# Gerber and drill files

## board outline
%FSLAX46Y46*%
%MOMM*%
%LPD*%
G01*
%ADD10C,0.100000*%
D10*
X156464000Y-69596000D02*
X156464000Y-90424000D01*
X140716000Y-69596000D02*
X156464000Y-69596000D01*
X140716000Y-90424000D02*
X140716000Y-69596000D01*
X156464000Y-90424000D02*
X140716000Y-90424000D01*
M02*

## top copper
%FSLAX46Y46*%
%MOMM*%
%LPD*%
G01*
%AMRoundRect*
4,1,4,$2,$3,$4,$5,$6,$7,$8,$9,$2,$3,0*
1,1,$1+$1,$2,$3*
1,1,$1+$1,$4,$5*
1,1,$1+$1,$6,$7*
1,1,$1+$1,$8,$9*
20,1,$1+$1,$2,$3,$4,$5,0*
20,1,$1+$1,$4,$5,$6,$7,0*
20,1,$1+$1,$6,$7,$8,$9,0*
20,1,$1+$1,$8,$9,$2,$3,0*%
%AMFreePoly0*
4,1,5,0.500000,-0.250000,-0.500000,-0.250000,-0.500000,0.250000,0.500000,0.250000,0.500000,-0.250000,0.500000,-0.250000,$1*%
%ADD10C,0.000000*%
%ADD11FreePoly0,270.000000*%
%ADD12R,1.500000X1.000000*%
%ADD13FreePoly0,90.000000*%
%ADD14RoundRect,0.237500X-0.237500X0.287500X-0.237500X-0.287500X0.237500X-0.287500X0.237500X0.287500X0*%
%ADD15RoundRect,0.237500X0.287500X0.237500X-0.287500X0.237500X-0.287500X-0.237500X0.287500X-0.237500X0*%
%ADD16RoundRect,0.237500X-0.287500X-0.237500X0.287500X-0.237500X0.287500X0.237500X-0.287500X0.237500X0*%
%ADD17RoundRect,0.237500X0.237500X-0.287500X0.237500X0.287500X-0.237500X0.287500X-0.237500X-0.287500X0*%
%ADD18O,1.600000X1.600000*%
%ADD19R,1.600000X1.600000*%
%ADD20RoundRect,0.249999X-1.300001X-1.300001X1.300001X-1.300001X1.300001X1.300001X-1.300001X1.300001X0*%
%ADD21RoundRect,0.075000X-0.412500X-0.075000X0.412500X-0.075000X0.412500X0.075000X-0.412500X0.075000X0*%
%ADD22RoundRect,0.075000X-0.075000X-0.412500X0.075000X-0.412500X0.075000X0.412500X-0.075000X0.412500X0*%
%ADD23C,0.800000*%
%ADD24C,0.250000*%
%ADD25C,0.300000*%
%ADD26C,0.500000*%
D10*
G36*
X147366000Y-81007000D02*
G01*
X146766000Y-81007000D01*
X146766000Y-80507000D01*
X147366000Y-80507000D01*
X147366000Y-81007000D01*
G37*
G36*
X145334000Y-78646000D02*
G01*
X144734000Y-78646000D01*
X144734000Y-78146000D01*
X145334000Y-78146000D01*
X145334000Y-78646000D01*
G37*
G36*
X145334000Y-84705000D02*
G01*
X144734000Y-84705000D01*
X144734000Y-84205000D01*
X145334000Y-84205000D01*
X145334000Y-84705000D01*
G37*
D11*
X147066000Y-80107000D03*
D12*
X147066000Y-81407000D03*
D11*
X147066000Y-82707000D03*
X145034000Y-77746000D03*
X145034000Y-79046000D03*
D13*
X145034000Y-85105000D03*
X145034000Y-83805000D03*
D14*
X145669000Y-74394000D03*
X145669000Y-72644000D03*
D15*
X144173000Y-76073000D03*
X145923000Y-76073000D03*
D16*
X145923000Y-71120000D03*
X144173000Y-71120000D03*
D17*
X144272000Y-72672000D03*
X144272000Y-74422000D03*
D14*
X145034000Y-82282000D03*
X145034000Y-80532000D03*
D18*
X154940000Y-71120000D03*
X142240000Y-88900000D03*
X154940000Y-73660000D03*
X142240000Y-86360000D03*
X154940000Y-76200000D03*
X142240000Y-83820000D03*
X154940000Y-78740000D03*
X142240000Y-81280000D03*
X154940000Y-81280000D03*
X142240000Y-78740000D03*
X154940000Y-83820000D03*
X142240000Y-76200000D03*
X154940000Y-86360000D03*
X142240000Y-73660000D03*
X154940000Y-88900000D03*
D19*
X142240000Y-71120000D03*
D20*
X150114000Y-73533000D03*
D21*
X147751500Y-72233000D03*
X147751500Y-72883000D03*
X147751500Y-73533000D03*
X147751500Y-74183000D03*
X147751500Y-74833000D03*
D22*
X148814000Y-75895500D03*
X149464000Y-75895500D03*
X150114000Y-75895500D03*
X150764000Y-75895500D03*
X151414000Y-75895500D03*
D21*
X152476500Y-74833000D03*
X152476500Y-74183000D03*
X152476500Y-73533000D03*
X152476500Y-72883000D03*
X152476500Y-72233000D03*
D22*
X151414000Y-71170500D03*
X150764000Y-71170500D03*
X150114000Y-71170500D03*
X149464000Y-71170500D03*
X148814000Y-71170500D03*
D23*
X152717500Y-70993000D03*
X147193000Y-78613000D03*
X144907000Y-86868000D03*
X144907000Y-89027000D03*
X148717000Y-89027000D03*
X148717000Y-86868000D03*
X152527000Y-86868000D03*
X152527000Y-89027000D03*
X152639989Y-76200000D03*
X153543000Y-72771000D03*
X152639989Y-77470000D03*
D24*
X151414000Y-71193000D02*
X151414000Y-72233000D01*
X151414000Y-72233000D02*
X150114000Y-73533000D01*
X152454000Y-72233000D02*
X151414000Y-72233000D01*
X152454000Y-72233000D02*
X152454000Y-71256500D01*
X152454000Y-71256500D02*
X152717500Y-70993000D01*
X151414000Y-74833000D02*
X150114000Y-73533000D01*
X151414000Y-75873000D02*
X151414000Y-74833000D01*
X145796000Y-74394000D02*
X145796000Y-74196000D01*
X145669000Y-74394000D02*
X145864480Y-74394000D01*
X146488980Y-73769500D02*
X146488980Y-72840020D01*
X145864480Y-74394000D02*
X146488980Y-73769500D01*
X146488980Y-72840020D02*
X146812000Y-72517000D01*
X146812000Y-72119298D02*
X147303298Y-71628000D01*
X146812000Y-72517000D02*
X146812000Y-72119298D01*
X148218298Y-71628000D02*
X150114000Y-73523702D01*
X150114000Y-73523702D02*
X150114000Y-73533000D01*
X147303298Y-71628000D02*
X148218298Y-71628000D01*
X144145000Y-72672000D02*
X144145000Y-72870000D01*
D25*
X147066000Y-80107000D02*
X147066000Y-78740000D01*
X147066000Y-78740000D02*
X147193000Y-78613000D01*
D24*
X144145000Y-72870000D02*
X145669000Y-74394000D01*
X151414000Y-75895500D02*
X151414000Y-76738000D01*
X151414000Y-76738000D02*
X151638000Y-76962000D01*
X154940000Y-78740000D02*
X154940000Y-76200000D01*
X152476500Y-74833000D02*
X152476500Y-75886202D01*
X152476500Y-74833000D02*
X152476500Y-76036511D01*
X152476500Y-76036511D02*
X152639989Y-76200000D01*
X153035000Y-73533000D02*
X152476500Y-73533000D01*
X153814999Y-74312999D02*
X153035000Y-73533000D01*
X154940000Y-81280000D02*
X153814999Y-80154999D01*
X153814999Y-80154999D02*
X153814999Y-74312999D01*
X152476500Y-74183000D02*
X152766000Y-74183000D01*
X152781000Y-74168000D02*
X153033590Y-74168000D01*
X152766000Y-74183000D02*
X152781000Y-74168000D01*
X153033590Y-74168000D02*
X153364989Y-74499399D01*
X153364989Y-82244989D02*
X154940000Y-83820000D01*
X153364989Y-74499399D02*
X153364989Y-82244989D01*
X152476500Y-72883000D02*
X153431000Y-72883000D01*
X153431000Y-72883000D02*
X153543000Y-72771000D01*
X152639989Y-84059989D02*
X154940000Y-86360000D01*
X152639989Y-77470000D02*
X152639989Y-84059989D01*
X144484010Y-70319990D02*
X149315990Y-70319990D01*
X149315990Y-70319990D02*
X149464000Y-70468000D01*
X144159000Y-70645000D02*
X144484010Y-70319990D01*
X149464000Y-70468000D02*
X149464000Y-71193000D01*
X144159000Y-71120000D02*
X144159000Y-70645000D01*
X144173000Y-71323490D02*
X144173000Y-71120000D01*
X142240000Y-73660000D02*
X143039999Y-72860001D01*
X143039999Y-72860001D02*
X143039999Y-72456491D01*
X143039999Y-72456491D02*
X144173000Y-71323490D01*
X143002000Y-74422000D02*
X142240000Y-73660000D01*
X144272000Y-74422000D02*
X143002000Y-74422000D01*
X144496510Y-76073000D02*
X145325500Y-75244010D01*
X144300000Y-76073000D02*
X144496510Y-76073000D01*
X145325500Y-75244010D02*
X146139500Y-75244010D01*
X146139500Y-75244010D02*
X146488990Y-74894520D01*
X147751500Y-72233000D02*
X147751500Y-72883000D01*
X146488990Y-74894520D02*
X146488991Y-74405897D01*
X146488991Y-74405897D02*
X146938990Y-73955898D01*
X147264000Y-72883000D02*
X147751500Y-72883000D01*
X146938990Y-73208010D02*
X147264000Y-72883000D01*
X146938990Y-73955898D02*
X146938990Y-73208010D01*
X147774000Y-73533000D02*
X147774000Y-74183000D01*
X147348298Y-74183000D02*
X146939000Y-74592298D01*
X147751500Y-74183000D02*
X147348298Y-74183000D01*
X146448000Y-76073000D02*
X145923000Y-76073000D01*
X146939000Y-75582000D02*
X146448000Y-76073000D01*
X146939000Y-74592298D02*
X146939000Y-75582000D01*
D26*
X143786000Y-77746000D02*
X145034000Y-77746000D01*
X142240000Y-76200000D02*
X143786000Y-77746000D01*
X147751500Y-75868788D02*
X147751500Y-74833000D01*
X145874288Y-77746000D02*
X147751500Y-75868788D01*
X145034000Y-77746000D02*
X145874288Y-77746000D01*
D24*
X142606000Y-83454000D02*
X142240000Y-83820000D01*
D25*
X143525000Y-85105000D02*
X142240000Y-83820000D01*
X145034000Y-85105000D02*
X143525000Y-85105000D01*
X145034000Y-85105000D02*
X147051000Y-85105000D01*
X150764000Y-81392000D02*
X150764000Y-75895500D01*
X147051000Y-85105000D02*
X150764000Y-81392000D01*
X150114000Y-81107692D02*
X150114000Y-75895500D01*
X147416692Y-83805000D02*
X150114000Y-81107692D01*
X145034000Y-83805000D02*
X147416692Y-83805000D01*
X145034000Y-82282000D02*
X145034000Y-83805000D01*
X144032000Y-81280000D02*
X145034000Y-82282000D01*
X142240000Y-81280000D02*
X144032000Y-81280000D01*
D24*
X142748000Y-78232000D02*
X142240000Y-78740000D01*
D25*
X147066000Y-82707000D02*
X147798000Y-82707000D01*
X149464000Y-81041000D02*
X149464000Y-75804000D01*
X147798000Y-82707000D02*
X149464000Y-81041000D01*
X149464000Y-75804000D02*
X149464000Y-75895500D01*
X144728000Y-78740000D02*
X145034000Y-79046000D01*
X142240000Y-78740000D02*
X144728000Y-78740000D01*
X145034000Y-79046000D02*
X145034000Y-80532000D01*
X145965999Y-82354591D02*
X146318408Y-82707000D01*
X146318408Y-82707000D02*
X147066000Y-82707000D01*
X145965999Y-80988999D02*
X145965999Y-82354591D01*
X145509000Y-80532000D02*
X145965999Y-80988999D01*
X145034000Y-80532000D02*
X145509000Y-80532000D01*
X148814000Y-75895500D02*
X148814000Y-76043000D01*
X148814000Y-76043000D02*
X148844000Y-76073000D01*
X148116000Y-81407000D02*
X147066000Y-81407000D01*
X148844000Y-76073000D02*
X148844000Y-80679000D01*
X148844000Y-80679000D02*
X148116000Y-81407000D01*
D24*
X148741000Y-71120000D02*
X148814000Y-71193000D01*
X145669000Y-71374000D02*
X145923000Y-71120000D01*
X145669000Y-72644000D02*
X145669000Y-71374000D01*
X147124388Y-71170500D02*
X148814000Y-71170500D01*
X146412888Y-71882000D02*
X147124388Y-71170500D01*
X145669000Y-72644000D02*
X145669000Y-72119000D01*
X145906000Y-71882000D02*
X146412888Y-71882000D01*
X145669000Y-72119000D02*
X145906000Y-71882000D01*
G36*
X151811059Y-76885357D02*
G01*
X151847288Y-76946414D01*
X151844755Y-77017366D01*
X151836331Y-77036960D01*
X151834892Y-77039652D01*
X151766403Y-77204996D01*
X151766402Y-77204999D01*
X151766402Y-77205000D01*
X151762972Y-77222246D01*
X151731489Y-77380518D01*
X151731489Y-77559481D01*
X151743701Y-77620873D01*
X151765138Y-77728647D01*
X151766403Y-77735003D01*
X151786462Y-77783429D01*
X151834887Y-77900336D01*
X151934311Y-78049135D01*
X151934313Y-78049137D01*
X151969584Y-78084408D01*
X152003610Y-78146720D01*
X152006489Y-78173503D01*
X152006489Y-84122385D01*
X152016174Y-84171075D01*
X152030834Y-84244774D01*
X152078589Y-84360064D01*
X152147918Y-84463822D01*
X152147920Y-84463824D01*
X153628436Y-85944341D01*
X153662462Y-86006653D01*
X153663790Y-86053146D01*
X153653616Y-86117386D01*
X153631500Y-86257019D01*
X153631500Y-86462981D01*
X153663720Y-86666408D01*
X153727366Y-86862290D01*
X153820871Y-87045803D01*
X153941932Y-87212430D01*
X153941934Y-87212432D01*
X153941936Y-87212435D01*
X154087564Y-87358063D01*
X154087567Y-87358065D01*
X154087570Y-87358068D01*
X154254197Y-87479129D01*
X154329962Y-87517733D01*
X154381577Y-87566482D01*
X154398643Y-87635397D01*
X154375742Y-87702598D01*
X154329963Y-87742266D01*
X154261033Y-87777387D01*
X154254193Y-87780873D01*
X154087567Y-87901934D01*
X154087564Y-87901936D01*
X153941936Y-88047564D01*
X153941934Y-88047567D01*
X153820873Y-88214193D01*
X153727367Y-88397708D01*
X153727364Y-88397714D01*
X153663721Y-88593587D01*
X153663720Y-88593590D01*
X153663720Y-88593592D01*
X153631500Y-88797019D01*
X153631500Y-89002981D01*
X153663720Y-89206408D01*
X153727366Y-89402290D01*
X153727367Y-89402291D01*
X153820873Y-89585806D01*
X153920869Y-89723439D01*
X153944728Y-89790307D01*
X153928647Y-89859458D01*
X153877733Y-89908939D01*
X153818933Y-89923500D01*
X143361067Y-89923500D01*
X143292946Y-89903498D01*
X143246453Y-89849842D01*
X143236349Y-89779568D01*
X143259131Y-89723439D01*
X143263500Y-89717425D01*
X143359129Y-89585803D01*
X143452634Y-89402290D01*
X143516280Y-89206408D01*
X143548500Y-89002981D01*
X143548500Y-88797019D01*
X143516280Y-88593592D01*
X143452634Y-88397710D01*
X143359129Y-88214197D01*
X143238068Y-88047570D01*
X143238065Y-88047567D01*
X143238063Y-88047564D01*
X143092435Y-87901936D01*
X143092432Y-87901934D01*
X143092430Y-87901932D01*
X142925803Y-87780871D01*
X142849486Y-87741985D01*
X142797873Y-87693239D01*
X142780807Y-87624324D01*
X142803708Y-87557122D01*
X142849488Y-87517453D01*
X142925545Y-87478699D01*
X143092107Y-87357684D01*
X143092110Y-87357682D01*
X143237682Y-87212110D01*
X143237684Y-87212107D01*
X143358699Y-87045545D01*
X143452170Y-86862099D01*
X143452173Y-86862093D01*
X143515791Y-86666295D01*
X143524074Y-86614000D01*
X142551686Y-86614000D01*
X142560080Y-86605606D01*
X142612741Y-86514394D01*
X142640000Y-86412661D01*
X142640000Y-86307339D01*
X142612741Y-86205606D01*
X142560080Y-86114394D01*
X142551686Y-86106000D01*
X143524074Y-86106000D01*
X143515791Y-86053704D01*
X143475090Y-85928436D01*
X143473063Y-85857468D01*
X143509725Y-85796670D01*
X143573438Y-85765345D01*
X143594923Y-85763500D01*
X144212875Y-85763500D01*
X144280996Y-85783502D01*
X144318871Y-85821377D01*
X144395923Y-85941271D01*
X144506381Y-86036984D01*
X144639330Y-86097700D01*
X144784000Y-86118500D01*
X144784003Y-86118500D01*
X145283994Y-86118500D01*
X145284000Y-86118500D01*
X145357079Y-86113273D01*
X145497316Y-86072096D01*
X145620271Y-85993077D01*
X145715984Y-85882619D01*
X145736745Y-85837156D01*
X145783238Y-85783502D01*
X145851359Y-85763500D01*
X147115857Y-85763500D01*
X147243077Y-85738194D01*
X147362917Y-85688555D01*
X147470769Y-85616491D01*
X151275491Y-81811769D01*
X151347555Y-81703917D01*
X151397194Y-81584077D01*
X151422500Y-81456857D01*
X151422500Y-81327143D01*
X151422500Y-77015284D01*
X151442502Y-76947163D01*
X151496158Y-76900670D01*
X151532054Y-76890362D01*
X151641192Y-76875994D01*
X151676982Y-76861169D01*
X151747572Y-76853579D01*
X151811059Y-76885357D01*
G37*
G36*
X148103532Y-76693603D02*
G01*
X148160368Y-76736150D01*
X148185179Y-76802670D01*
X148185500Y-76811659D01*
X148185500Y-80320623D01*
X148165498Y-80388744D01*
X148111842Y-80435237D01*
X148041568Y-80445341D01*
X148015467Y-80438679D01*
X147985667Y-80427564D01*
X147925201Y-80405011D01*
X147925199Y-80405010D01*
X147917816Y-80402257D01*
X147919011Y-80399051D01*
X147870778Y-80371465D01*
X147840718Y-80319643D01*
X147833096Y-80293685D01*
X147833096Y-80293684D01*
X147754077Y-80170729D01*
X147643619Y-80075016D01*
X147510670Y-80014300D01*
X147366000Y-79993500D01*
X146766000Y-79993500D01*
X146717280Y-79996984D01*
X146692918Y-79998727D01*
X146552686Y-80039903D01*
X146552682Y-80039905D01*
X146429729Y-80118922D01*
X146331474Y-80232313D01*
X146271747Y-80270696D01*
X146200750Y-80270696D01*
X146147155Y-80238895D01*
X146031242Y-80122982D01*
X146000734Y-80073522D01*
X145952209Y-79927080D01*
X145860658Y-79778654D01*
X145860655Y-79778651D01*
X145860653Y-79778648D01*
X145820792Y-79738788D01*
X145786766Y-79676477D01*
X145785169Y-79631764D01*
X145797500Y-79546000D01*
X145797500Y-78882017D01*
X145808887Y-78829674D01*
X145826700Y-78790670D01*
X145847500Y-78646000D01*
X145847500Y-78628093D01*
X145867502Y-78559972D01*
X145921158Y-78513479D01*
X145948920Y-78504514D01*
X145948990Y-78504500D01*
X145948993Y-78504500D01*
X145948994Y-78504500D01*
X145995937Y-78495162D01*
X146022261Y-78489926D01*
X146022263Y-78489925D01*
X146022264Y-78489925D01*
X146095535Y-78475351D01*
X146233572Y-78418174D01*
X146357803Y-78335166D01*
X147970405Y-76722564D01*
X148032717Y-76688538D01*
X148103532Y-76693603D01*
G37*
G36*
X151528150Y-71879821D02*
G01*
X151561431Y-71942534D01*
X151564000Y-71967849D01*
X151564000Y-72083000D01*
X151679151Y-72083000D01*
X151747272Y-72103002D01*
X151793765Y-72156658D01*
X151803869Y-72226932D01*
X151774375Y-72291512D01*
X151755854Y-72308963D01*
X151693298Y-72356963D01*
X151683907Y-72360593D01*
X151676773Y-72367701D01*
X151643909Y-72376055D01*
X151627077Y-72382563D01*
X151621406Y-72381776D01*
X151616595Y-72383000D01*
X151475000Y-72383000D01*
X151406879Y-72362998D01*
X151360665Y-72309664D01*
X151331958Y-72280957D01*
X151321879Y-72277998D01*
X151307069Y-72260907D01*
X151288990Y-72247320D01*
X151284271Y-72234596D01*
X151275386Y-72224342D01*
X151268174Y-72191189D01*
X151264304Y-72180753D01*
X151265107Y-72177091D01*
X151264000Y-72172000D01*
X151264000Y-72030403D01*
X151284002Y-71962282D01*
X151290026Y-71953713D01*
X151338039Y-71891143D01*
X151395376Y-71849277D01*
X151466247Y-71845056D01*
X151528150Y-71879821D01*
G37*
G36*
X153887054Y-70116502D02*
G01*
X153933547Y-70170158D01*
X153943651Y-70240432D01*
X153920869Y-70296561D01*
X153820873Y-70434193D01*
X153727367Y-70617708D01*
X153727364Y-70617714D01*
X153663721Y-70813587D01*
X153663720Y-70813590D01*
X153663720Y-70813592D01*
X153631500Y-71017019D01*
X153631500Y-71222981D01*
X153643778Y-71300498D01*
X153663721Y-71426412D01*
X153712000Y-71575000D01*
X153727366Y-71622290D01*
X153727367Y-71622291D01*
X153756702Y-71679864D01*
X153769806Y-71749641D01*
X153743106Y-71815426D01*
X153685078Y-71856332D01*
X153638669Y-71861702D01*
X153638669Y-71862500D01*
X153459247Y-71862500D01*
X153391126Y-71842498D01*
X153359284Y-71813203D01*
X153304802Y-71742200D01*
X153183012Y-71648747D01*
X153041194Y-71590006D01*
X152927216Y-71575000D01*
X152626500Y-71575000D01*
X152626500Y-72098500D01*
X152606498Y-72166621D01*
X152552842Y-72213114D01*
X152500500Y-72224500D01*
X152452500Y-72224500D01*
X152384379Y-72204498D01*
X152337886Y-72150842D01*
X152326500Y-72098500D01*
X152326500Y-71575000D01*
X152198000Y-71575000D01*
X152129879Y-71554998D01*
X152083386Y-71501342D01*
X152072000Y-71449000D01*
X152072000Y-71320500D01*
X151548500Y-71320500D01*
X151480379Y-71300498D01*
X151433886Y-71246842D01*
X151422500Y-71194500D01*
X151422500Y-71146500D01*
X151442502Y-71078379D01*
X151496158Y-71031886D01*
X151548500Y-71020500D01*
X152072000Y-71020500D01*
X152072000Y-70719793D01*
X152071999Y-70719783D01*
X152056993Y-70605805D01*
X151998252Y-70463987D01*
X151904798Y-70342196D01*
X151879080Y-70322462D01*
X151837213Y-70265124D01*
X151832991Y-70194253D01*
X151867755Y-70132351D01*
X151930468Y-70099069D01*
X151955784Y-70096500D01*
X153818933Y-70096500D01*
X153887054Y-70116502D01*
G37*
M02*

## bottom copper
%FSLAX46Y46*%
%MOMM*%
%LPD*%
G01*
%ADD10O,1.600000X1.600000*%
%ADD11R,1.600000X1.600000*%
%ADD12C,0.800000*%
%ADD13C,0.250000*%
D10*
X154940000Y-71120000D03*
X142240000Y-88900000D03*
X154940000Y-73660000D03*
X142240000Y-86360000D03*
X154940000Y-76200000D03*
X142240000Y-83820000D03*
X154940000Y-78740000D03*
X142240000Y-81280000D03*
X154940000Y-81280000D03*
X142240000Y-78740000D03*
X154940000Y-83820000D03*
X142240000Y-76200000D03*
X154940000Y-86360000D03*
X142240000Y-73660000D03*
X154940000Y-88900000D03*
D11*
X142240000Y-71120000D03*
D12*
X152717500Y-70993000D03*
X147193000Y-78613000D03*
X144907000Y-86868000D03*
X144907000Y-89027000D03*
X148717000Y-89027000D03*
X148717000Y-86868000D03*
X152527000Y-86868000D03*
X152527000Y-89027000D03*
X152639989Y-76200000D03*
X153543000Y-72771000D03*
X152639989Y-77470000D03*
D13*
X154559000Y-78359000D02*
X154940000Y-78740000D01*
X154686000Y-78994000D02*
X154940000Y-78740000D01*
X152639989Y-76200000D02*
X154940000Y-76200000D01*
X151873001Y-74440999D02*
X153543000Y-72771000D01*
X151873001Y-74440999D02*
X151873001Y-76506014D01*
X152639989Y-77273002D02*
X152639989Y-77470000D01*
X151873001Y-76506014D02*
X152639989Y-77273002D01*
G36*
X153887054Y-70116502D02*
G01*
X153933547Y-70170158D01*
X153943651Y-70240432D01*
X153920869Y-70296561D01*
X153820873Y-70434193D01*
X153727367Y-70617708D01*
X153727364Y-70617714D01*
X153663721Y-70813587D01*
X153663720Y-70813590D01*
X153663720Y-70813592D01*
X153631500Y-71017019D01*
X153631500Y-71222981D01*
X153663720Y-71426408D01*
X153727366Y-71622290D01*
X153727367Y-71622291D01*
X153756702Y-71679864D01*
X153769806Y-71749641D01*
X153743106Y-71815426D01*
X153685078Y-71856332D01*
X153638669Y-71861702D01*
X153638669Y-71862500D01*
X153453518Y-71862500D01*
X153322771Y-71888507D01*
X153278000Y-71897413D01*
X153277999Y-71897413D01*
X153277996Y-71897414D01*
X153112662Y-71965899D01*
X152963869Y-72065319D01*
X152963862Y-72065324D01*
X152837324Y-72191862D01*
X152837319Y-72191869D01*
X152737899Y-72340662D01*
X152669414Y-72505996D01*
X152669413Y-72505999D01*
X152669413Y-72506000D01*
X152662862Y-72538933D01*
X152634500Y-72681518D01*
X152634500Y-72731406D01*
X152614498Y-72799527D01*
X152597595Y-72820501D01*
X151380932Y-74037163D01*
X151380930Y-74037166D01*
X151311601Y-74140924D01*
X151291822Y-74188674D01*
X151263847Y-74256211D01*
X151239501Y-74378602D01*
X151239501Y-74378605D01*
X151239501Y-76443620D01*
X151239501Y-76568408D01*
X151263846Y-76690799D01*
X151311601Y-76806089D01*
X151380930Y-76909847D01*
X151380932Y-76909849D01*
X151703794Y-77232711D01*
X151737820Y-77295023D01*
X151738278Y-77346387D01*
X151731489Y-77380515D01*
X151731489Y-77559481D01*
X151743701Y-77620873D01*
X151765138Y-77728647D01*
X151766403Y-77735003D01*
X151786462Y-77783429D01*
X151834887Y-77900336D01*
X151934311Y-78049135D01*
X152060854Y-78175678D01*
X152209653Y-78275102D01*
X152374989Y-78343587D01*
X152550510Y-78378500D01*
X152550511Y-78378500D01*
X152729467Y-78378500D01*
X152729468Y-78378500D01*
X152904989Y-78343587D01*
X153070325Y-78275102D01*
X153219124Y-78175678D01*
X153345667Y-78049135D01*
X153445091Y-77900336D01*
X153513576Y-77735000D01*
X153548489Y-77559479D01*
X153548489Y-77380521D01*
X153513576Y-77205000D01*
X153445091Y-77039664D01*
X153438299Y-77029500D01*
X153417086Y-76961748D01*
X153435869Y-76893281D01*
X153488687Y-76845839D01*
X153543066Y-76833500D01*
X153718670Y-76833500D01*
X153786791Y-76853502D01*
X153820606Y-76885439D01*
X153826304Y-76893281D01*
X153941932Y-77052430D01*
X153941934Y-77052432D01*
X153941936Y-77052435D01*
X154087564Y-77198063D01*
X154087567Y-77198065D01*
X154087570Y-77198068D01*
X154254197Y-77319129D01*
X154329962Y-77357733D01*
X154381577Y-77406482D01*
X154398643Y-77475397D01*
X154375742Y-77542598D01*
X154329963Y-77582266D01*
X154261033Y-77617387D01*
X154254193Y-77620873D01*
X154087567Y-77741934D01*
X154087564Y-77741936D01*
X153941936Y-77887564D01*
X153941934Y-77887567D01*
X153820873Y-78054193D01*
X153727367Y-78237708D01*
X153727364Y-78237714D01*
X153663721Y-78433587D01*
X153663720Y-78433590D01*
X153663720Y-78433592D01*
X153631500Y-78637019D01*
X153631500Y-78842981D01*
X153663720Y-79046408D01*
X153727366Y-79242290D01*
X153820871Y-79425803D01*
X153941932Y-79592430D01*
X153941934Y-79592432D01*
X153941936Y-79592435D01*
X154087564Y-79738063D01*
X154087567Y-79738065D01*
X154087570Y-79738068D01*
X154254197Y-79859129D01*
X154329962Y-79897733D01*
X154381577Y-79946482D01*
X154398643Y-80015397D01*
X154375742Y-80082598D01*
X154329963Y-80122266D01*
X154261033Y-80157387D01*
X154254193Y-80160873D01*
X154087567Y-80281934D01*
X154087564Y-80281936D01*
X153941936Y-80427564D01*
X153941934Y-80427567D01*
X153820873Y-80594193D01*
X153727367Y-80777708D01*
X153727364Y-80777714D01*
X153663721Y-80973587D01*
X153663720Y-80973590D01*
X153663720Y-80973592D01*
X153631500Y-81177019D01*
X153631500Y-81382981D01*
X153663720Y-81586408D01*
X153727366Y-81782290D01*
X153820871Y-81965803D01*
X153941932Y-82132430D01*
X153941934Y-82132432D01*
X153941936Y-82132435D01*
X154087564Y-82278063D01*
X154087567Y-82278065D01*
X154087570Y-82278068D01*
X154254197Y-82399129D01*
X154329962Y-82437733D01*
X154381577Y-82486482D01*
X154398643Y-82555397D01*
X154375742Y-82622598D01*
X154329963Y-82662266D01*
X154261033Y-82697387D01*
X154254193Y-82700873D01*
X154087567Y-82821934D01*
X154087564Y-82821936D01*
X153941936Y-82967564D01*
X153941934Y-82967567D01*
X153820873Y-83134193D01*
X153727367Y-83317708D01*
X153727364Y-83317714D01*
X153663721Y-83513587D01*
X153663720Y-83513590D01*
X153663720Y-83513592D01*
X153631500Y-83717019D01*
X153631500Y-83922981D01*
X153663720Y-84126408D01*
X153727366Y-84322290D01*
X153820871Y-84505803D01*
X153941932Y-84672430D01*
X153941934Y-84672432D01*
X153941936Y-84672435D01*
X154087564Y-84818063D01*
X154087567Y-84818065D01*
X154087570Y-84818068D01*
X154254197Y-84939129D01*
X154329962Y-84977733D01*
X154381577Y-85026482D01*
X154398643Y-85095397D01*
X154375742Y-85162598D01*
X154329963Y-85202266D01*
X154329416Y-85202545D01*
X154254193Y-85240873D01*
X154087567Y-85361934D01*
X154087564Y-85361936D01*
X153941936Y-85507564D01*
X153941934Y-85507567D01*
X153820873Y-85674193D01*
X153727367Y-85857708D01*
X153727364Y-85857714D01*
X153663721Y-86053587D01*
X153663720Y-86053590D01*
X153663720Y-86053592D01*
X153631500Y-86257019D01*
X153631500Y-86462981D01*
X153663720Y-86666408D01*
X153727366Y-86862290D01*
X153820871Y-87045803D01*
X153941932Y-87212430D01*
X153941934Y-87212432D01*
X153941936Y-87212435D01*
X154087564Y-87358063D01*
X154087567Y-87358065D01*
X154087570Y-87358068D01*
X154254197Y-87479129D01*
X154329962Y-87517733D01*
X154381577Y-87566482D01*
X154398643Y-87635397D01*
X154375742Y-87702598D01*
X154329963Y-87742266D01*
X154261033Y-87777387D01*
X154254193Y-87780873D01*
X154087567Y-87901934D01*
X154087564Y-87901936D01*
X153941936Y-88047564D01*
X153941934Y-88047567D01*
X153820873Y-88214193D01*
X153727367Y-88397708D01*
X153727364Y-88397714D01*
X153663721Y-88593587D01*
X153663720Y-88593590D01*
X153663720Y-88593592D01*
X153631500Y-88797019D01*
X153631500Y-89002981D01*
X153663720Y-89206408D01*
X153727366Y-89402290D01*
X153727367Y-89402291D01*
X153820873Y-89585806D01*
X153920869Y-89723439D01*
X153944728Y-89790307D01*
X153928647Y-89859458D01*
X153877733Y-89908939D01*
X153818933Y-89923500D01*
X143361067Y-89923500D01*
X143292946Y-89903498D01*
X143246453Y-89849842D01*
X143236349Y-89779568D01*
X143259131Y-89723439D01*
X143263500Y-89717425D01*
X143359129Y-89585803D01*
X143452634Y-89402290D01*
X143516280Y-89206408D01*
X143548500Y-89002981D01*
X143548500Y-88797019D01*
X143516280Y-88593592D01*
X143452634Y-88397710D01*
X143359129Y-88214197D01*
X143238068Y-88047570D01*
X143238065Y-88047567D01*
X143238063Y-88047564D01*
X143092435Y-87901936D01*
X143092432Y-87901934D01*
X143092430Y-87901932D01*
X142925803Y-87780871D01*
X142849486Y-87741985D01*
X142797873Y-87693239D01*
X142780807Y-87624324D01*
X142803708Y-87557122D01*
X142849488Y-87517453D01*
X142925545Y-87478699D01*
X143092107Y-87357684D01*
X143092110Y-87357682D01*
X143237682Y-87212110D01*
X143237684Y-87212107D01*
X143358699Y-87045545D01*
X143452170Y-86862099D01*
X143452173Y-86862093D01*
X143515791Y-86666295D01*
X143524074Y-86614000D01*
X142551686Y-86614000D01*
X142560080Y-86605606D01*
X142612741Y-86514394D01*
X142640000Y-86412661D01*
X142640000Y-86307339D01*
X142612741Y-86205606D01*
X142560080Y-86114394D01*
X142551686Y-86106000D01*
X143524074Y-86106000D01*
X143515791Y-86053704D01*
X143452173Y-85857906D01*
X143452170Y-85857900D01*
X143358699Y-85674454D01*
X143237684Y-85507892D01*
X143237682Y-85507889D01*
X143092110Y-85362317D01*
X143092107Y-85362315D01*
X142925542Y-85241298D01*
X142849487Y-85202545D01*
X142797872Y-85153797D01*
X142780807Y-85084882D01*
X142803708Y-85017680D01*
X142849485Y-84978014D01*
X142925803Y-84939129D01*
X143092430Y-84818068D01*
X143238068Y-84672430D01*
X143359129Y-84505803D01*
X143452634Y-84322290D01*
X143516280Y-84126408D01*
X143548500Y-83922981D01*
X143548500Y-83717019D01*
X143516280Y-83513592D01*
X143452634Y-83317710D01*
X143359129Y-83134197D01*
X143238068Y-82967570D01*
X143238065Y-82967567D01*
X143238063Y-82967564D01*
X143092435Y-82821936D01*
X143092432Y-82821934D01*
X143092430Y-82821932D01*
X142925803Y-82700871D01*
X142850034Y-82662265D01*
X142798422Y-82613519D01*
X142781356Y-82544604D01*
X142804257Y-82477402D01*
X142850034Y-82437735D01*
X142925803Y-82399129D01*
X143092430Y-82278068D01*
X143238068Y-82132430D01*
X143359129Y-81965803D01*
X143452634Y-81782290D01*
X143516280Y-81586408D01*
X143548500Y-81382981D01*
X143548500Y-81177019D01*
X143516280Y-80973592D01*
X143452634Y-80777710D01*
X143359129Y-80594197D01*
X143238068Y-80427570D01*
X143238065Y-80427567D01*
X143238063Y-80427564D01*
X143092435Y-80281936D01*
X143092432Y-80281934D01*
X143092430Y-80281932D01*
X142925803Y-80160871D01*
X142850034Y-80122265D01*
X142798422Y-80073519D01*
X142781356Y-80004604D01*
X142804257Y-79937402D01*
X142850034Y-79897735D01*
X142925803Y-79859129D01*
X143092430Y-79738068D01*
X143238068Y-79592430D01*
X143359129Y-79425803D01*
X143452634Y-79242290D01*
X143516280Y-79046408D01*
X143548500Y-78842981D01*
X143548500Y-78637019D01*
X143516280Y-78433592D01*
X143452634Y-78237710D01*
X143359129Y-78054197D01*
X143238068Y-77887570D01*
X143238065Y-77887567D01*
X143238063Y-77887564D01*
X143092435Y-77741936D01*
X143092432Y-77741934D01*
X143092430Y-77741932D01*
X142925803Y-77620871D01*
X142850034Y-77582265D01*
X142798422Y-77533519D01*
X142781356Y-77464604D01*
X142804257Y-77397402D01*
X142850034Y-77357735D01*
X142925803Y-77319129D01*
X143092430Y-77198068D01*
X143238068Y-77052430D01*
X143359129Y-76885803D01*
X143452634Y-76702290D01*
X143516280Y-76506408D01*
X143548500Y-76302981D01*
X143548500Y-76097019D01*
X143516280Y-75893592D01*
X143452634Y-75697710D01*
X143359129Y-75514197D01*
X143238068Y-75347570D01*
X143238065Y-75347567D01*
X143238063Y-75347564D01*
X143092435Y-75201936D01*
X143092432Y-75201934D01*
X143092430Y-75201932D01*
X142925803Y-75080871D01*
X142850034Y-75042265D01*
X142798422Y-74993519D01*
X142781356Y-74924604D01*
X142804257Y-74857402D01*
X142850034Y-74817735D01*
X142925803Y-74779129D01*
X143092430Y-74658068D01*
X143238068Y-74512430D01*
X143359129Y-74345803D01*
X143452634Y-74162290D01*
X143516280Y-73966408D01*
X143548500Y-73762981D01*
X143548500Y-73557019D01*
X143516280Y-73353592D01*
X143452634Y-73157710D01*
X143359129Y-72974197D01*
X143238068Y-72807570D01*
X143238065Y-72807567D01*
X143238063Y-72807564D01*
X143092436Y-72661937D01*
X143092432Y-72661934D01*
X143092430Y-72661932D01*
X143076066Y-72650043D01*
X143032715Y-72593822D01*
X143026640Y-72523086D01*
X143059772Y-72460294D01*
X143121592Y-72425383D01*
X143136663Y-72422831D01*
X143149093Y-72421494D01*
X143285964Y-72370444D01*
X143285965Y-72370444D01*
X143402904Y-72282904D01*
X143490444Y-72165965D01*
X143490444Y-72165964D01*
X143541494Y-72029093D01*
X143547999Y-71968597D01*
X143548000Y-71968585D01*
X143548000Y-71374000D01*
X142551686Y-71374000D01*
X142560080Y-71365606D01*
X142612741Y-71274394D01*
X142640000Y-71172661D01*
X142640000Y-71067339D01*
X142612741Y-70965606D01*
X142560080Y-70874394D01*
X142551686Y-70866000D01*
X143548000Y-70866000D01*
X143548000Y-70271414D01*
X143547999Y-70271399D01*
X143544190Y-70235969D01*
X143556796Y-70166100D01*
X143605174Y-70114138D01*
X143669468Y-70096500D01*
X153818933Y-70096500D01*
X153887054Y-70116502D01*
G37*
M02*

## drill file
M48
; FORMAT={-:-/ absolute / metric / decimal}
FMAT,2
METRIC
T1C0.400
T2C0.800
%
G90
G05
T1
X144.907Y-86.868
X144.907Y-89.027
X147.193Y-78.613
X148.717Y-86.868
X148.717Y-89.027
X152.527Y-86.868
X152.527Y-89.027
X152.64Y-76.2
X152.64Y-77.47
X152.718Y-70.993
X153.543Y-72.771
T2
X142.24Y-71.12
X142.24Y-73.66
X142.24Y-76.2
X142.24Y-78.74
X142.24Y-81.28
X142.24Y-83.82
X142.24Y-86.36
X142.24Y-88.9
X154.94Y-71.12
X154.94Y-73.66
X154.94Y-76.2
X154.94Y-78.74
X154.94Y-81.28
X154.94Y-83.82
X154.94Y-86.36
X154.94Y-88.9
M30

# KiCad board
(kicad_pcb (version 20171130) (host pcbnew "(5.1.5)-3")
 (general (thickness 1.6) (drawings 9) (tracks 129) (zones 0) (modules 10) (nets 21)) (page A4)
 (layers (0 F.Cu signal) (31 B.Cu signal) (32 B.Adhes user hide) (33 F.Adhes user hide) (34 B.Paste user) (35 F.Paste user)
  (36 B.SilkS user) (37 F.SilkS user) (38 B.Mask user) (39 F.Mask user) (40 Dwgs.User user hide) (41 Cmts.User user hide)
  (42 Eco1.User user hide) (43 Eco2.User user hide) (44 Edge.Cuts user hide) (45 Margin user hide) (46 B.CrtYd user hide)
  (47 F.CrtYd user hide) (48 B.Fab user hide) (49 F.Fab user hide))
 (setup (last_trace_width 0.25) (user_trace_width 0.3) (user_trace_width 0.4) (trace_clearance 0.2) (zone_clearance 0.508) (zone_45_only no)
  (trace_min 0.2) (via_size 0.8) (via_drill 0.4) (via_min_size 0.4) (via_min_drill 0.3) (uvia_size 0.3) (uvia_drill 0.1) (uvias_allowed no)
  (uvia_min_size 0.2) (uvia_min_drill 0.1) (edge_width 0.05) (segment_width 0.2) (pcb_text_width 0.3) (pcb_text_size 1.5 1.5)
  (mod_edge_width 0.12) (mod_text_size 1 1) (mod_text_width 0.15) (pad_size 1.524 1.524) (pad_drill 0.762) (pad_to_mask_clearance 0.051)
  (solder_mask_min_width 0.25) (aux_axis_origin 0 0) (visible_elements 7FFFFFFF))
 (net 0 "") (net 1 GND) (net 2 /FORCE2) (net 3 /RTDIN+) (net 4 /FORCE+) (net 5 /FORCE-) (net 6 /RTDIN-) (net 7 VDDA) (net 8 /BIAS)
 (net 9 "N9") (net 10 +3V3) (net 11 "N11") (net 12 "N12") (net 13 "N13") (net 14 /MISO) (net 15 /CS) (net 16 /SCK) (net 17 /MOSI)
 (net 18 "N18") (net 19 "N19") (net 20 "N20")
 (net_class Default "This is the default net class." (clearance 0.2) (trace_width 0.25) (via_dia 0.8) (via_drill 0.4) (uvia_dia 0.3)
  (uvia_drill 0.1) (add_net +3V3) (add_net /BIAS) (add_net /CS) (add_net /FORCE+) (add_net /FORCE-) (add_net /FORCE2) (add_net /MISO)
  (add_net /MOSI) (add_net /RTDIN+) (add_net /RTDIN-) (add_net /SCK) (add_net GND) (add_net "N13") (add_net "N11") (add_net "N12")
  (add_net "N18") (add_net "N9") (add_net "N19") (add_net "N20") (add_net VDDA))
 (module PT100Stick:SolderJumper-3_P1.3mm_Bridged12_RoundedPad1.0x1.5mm (layer F.Cu) (at 147.066 81.407 270)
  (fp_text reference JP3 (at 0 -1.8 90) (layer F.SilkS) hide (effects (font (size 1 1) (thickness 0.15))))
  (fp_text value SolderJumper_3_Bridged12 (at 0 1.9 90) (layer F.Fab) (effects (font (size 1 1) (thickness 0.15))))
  (fp_poly (pts (xy -0.9 -0.3) (xy -0.4 -0.3) (xy -0.4 0.3) (xy -0.9 0.3)) (layer F.Cu) (width 0))
  (pad 1 smd custom (at -1.3 0 270) (size 1 0.5) (layers F.Cu F.Mask) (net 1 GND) (zone_connect 2)
   (options (clearance outline) (anchor rect)) (primitives))
  (pad 2 smd rect (at 0 0 270) (size 1 1.5) (layers F.Cu F.Mask) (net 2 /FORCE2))
  (pad 3 smd custom (at 1.3 0 270) (size 1 0.5) (layers F.Cu F.Mask) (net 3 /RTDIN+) (zone_connect 2)
   (options (clearance outline) (anchor rect)) (primitives)))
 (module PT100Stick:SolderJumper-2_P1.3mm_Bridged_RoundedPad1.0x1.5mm (layer F.Cu) (at 145.034 78.396 270)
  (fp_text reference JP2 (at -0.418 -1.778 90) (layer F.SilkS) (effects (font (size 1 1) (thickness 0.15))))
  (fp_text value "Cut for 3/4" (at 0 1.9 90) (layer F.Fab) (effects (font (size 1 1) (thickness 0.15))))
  (fp_poly (pts (xy 0.25 -0.3) (xy -0.25 -0.3) (xy -0.25 0.3) (xy 0.25 0.3)) (layer F.Cu) (width 0))
  (pad 1 smd custom (at -0.65 0 270) (size 1 0.5) (layers F.Cu F.Mask) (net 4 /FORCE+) (zone_connect 2)
   (options (clearance outline) (anchor rect)) (primitives))
  (pad 2 smd custom (at 0.65 0 270) (size 1 0.5) (layers F.Cu F.Mask) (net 3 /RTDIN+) (zone_connect 2)
   (options (clearance outline) (anchor rect)) (primitives)))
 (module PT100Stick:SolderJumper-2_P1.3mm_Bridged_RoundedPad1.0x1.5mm (layer F.Cu) (at 145.034 84.455 90)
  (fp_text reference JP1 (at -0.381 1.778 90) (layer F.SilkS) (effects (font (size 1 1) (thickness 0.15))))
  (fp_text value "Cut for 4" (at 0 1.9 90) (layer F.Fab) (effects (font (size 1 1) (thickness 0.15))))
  (fp_poly (pts (xy 0.25 -0.3) (xy -0.25 -0.3) (xy -0.25 0.3) (xy 0.25 0.3)) (layer F.Cu) (width 0))
  (pad 1 smd custom (at -0.65 0 90) (size 1 0.5) (layers F.Cu F.Mask) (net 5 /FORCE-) (zone_connect 2)
   (options (clearance outline) (anchor rect)) (primitives))
  (pad 2 smd custom (at 0.65 0 90) (size 1 0.5) (layers F.Cu F.Mask) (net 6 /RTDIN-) (zone_connect 2)
   (options (clearance outline) (anchor rect)) (primitives)))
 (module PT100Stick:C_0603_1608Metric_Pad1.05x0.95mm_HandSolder (layer F.Cu) (at 145.669 73.519 270)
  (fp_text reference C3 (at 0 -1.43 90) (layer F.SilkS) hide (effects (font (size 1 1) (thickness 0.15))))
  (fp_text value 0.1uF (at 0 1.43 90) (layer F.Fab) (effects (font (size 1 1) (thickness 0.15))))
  (pad 2 smd roundrect (at 0.875 0 270) (size 1.05 0.95) (layers F.Cu F.Paste F.Mask) (roundrect_rratio 0.25) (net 1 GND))
  (pad 1 smd roundrect (at -0.875 0 270) (size 1.05 0.95) (layers F.Cu F.Paste F.Mask) (roundrect_rratio 0.25) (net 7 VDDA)))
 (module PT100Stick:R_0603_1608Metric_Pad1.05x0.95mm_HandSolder (layer F.Cu) (at 145.048 76.073 180)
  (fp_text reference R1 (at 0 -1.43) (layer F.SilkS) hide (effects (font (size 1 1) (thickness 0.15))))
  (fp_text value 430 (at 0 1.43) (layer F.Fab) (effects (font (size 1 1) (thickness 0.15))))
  (pad 2 smd roundrect (at 0.875 0 180) (size 1.05 0.95) (layers F.Cu F.Paste F.Mask) (roundrect_rratio 0.25) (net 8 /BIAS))
  (pad 1 smd roundrect (at -0.875 0 180) (size 1.05 0.95) (layers F.Cu F.Paste F.Mask) (roundrect_rratio 0.25) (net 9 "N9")))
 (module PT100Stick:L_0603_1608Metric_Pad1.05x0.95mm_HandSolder (layer F.Cu) (at 145.048 71.12)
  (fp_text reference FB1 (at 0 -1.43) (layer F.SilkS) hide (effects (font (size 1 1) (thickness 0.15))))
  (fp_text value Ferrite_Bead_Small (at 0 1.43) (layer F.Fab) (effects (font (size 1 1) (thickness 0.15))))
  (pad 2 smd roundrect (at 0.875 0) (size 1.05 0.95) (layers F.Cu F.Paste F.Mask) (roundrect_rratio 0.25) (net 7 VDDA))
  (pad 1 smd roundrect (at -0.875 0) (size 1.05 0.95) (layers F.Cu F.Paste F.Mask) (roundrect_rratio 0.25) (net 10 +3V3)))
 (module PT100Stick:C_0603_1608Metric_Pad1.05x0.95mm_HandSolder (layer F.Cu) (at 144.272 73.547 90)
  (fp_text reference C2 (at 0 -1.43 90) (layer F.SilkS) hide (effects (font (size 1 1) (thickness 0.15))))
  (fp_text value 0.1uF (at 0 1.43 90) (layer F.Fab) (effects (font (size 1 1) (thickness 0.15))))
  (pad 2 smd roundrect (at 0.875 0 90) (size 1.05 0.95) (layers F.Cu F.Paste F.Mask) (roundrect_rratio 0.25) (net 1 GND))
  (pad 1 smd roundrect (at -0.875 0 90) (size 1.05 0.95) (layers F.Cu F.Paste F.Mask) (roundrect_rratio 0.25) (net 10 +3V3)))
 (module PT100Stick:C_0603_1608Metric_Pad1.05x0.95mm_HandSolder (layer F.Cu) (at 145.034 81.407 270)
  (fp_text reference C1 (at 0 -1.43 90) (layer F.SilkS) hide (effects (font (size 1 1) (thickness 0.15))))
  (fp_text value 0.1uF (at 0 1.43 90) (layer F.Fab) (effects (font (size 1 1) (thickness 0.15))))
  (pad 2 smd roundrect (at 0.875 0 270) (size 1.05 0.95) (layers F.Cu F.Paste F.Mask) (roundrect_rratio 0.25) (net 6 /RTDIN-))
  (pad 1 smd roundrect (at -0.875 0 270) (size 1.05 0.95) (layers F.Cu F.Paste F.Mask) (roundrect_rratio 0.25) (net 3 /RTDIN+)))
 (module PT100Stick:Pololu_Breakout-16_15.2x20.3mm (layer F.Cu) (at 142.24 71.12)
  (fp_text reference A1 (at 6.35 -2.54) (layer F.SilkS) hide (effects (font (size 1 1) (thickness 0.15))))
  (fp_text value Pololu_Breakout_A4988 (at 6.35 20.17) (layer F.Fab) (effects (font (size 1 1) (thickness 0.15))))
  (pad 16 thru_hole oval (at 12.7 0) (size 1.6 1.6) (drill 0.8) (layers *.Cu *.Mask) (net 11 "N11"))
  (pad 8 thru_hole oval (at 0 17.78) (size 1.6 1.6) (drill 0.8) (layers *.Cu *.Mask) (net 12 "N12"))
  (pad 15 thru_hole oval (at 12.7 2.54) (size 1.6 1.6) (drill 0.8) (layers *.Cu *.Mask) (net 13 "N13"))
  (pad 7 thru_hole oval (at 0 15.24) (size 1.6 1.6) (drill 0.8) (layers *.Cu *.Mask) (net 1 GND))
  (pad 14 thru_hole oval (at 12.7 5.08) (size 1.6 1.6) (drill 0.8) (layers *.Cu *.Mask) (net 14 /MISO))
  (pad 6 thru_hole oval (at 0 12.7) (size 1.6 1.6) (drill 0.8) (layers *.Cu *.Mask) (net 5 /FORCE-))
  (pad 13 thru_hole oval (at 12.7 7.62) (size 1.6 1.6) (drill 0.8) (layers *.Cu *.Mask) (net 14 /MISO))
  (pad 5 thru_hole oval (at 0 10.16) (size 1.6 1.6) (drill 0.8) (layers *.Cu *.Mask) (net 6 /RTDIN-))
  (pad 12 thru_hole oval (at 12.7 10.16) (size 1.6 1.6) (drill 0.8) (layers *.Cu *.Mask) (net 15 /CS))
  (pad 4 thru_hole oval (at 0 7.62) (size 1.6 1.6) (drill 0.8) (layers *.Cu *.Mask) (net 3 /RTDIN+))
  (pad 11 thru_hole oval (at 12.7 12.7) (size 1.6 1.6) (drill 0.8) (layers *.Cu *.Mask) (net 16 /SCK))
  (pad 3 thru_hole oval (at 0 5.08) (size 1.6 1.6) (drill 0.8) (layers *.Cu *.Mask) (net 4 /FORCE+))
  (pad 10 thru_hole oval (at 12.7 15.24) (size 1.6 1.6) (drill 0.8) (layers *.Cu *.Mask) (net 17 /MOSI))
  (pad 2 thru_hole oval (at 0 2.54) (size 1.6 1.6) (drill 0.8) (layers *.Cu *.Mask) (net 10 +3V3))
  (pad 9 thru_hole oval (at 12.7 17.78) (size 1.6 1.6) (drill 0.8) (layers *.Cu *.Mask) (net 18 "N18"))
  (pad 1 thru_hole rect (at 0 0) (size 1.6 1.6) (drill 0.8) (layers *.Cu *.Mask) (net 1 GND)))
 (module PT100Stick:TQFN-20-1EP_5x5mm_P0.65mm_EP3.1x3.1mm (layer F.Cu) (at 150.114 73.533)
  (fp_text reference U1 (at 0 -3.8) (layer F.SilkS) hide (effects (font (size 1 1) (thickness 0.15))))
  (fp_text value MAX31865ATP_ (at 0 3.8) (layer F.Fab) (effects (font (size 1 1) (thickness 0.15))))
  (pad 21 smd roundrect (at 0 0) (size 3.1 3.1) (layers F.Cu F.Mask) (roundrect_rratio 0.08064499999999999) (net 1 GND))
  (pad "" smd roundrect (at -0.775 -0.775) (size 1.25 1.25) (layers F.Paste) (roundrect_rratio 0.2))
  (pad "" smd roundrect (at -0.775 0.775) (size 1.25 1.25) (layers F.Paste) (roundrect_rratio 0.2))
  (pad "" smd roundrect (at 0.775 -0.775) (size 1.25 1.25) (layers F.Paste) (roundrect_rratio 0.2))
  (pad "" smd roundrect (at 0.775 0.775) (size 1.25 1.25) (layers F.Paste) (roundrect_rratio 0.2))
  (pad 1 smd roundrect (at -2.3625 -1.3) (size 0.975 0.3) (layers F.Cu F.Paste F.Mask) (roundrect_rratio 0.25) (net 8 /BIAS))
  (pad 2 smd roundrect (at -2.3625 -0.65) (size 0.975 0.3) (layers F.Cu F.Paste F.Mask) (roundrect_rratio 0.25) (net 8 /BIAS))
  (pad 3 smd roundrect (at -2.3625 0) (size 0.975 0.3) (layers F.Cu F.Paste F.Mask) (roundrect_rratio 0.25) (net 9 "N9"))
  (pad 4 smd roundrect (at -2.3625 0.65) (size 0.975 0.3) (layers F.Cu F.Paste F.Mask) (roundrect_rratio 0.25) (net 9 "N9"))
  (pad 5 smd roundrect (at -2.3625 1.3) (size 0.975 0.3) (layers F.Cu F.Paste F.Mask) (roundrect_rratio 0.25) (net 4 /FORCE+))
  (pad 6 smd roundrect (at -1.3 2.3625) (size 0.3 0.975) (layers F.Cu F.Paste F.Mask) (roundrect_rratio 0.25) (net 2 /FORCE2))
  (pad 7 smd roundrect (at -0.65 2.3625) (size 0.3 0.975) (layers F.Cu F.Paste F.Mask) (roundrect_rratio 0.25) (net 3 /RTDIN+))
  (pad 8 smd roundrect (at 0 2.3625) (size 0.3 0.975) (layers F.Cu F.Paste F.Mask) (roundrect_rratio 0.25) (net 6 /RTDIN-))
  (pad 9 smd roundrect (at 0.65 2.3625) (size 0.3 0.975) (layers F.Cu F.Paste F.Mask) (roundrect_rratio 0.25) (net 5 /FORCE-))
  (pad 10 smd roundrect (at 1.3 2.3625) (size 0.3 0.975) (layers F.Cu F.Paste F.Mask) (roundrect_rratio 0.25) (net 1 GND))
  (pad 11 smd roundrect (at 2.3625 1.3) (size 0.975 0.3) (layers F.Cu F.Paste F.Mask) (roundrect_rratio 0.25) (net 14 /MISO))
  (pad 12 smd roundrect (at 2.3625 0.65) (size 0.975 0.3) (layers F.Cu F.Paste F.Mask) (roundrect_rratio 0.25) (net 16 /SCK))
  (pad 13 smd roundrect (at 2.3625 0) (size 0.975 0.3) (layers F.Cu F.Paste F.Mask) (roundrect_rratio 0.25) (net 15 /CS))
  (pad 14 smd roundrect (at 2.3625 -0.65) (size 0.975 0.3) (layers F.Cu F.Paste F.Mask) (roundrect_rratio 0.25) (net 17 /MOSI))
  (pad 15 smd roundrect (at 2.3625 -1.3) (size 0.975 0.3) (layers F.Cu F.Paste F.Mask) (roundrect_rratio 0.25) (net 1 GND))
  (pad 16 smd roundrect (at 1.3 -2.3625) (size 0.3 0.975) (layers F.Cu F.Paste F.Mask) (roundrect_rratio 0.25) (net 1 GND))
  (pad 17 smd roundrect (at 0.65 -2.3625) (size 0.3 0.975) (layers F.Cu F.Paste F.Mask) (roundrect_rratio 0.25) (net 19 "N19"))
  (pad 18 smd roundrect (at 0 -2.3625) (size 0.3 0.975) (layers F.Cu F.Paste F.Mask) (roundrect_rratio 0.25) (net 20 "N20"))
  (pad 19 smd roundrect (at -0.65 -2.3625) (size 0.3 0.975) (layers F.Cu F.Paste F.Mask) (roundrect_rratio 0.25) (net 10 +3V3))
  (pad 20 smd roundrect (at -1.3 -2.3625) (size 0.3 0.975) (layers F.Cu F.Paste F.Mask) (roundrect_rratio 0.25) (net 7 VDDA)))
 (gr_line (start 156.464 69.596) (end 156.464 90.424) (layer Edge.Cuts) (width 0.1))
 (gr_line (start 140.716 69.596) (end 156.464 69.596) (layer Edge.Cuts) (width 0.1))
 (gr_line (start 140.716 90.424) (end 140.716 69.596) (layer Edge.Cuts) (width 0.1))
 (gr_line (start 156.464 90.424) (end 140.716 90.424) (layer Edge.Cuts) (width 0.1))
 (segment (start 151.414 71.193) (end 151.414 72.233) (width 0.25) (layer F.Cu) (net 1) (status 30))
 (segment (start 151.414 72.233) (end 150.114 73.533) (width 0.25) (layer F.Cu) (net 1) (status 30))
 (segment (start 152.454 72.233) (end 151.414 72.233) (width 0.25) (layer F.Cu) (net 1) (status 30))
 (via (at 152.7175 70.993) (size 0.8) (drill 0.4) (layers F.Cu B.Cu) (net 1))
 (segment (start 152.454 72.233) (end 152.454 71.2565) (width 0.25) (layer F.Cu) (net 1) (status 10))
 (segment (start 152.454 71.2565) (end 152.7175 70.993) (width 0.25) (layer F.Cu) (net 1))
 (segment (start 151.414 74.833) (end 150.114 73.533) (width 0.25) (layer F.Cu) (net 1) (status 30))
 (segment (start 151.414 75.873) (end 151.414 74.833) (width 0.25) (layer F.Cu) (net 1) (status 30))
 (segment (start 145.796 74.394) (end 145.796 74.196) (width 0.25) (layer F.Cu) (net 1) (status 30))
 (segment (start 145.669 74.394) (end 145.86448 74.394) (width 0.25) (layer F.Cu) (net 1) (status 30))
 (segment (start 146.48898 73.7695) (end 146.48898 72.84002) (width 0.25) (layer F.Cu) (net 1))
 (segment (start 145.86448 74.394) (end 146.48898 73.7695) (width 0.25) (layer F.Cu) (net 1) (status 10))
 (segment (start 146.48898 72.84002) (end 146.812 72.517) (width 0.25) (layer F.Cu) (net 1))
 (segment (start 146.812 72.119298) (end 147.303298 71.628) (width 0.25) (layer F.Cu) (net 1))
 (segment (start 146.812 72.517) (end 146.812 72.119298) (width 0.25) (layer F.Cu) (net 1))
 (segment (start 148.218298 71.628) (end 150.114 73.523702) (width 0.25) (layer F.Cu) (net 1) (status 20))
 (segment (start 150.114 73.523702) (end 150.114 73.533) (width 0.25) (layer F.Cu) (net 1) (status 30))
 (segment (start 147.303298 71.628) (end 148.218298 71.628) (width 0.25) (layer F.Cu) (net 1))
 (segment (start 144.145 72.672) (end 144.145 72.87) (width 0.25) (layer F.Cu) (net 1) (status 30))
 (via (at 147.193 78.613) (size 0.8) (drill 0.4) (layers F.Cu B.Cu) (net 1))
 (segment (start 147.066 80.107) (end 147.066 78.74) (width 0.3) (layer F.Cu) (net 1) (status 10))
 (segment (start 147.066 78.74) (end 147.193 78.613) (width 0.3) (layer F.Cu) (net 1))
 (via (at 144.907 86.868) (size 0.8) (drill 0.4) (layers F.Cu B.Cu) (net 1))
 (via (at 144.907 89.027) (size 0.8) (drill 0.4) (layers F.Cu B.Cu) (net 1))
 (via (at 148.717 89.027) (size 0.8) (drill 0.4) (layers F.Cu B.Cu) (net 1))
 (via (at 148.717 86.868) (size 0.8) (drill 0.4) (layers F.Cu B.Cu) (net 1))
 (via (at 152.527 86.868) (size 0.8) (drill 0.4) (layers F.Cu B.Cu) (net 1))
 (via (at 152.527 89.027) (size 0.8) (drill 0.4) (layers F.Cu B.Cu) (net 1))
 (segment (start 144.145 72.87) (end 145.669 74.394) (width 0.25) (layer F.Cu) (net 1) (status 30))
 (segment (start 151.414 75.8955) (end 151.414 76.738) (width 0.25) (layer F.Cu) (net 1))
 (segment (start 151.414 76.738) (end 151.638 76.962) (width 0.25) (layer F.Cu) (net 1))
 (segment (start 154.94 78.74) (end 154.94 76.2) (width 0.25) (layer F.Cu) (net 14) (status 30))
 (segment (start 154.559 78.359) (end 154.94 78.74) (width 0.25) (layer B.Cu) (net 14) (status 30))
 (segment (start 152.4765 74.833) (end 152.4765 75.886202) (width 0.25) (layer F.Cu) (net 14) (status 10))
 (segment (start 154.686 78.994) (end 154.94 78.74) (width 0.25) (layer B.Cu) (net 14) (status 30))
 (via (at 152.639989 76.2) (size 0.8) (drill 0.4) (layers F.Cu B.Cu) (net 14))
 (segment (start 152.4765 74.833) (end 152.4765 76.036511) (width 0.25) (layer F.Cu) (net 14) (status 10))
 (segment (start 152.4765 76.036511) (end 152.639989 76.2) (width 0.25) (layer F.Cu) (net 14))
 (segment (start 152.639989 76.2) (end 154.94 76.2) (width 0.25) (layer B.Cu) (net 14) (status 20))
 (segment (start 153.035 73.533) (end 152.4765 73.533) (width 0.25) (layer F.Cu) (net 15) (status 20))
 (segment (start 153.814999 74.312999) (end 153.035 73.533) (width 0.25) (layer F.Cu) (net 15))
 (segment (start 154.94 81.28) (end 153.814999 80.154999) (width 0.25) (layer F.Cu) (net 15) (status 10))
 (segment (start 153.814999 80.154999) (end 153.814999 74.312999) (width 0.25) (layer F.Cu) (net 15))
 (segment (start 152.4765 74.183) (end 152.766 74.183) (width 0.25) (layer F.Cu) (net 16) (status 30))
 (segment (start 152.781 74.168) (end 153.03359 74.168) (width 0.25) (layer F.Cu) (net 16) (status 10))
 (segment (start 152.766 74.183) (end 152.781 74.168) (width 0.25) (layer F.Cu) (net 16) (status 30))
 (segment (start 153.03359 74.168) (end 153.364989 74.499399) (width 0.25) (layer F.Cu) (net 16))
 (segment (start 153.364989 82.244989) (end 154.94 83.82) (width 0.25) (layer F.Cu) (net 16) (status 20))
 (segment (start 153.364989 74.499399) (end 153.364989 82.244989) (width 0.25) (layer F.Cu) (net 16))
 (via (at 153.543 72.771) (size 0.8) (drill 0.4) (layers F.Cu B.Cu) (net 17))
 (segment (start 152.4765 72.883) (end 153.431 72.883) (width 0.25) (layer F.Cu) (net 17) (status 10))
 (segment (start 153.431 72.883) (end 153.543 72.771) (width 0.25) (layer F.Cu) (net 17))
 (segment (start 151.873001 74.440999) (end 153.543 72.771) (width 0.25) (layer B.Cu) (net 17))
 (via (at 152.639989 77.47) (size 0.8) (drill 0.4) (layers F.Cu B.Cu) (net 17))
 (segment (start 151.873001 74.440999) (end 151.873001 76.506014) (width 0.25) (layer B.Cu) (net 17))
 (segment (start 152.639989 77.273002) (end 152.639989 77.47) (width 0.25) (layer B.Cu) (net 17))
 (segment (start 151.873001 76.506014) (end 152.639989 77.273002) (width 0.25) (layer B.Cu) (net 17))
 (segment (start 152.639989 84.059989) (end 154.94 86.36) (width 0.25) (layer F.Cu) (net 17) (status 20))
 (segment (start 152.639989 77.47) (end 152.639989 84.059989) (width 0.25) (layer F.Cu) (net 17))
 (segment (start 144.48401 70.31999) (end 149.31599 70.31999) (width 0.25) (layer F.Cu) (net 10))
 (segment (start 149.31599 70.31999) (end 149.464 70.468) (width 0.25) (layer F.Cu) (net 10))
 (segment (start 144.159 70.645) (end 144.48401 70.31999) (width 0.25) (layer F.Cu) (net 10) (status 10))
 (segment (start 149.464 70.468) (end 149.464 71.193) (width 0.25) (layer F.Cu) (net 10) (status 20))
 (segment (start 144.159 71.12) (end 144.159 70.645) (width 0.25) (layer F.Cu) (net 10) (status 30))
 (segment (start 144.173 71.32349) (end 144.173 71.12) (width 0.25) (layer F.Cu) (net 10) (status 30))
 (segment (start 142.24 73.66) (end 143.039999 72.860001) (width 0.25) (layer F.Cu) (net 10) (status 10))
 (segment (start 143.039999 72.860001) (end 143.039999 72.456491) (width 0.25) (layer F.Cu) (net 10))
 (segment (start 143.039999 72.456491) (end 144.173 71.32349) (width 0.25) (layer F.Cu) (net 10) (status 20))
 (segment (start 143.002 74.422) (end 142.24 73.66) (width 0.25) (layer F.Cu) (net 10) (status 20))
 (segment (start 144.272 74.422) (end 143.002 74.422) (width 0.25) (layer F.Cu) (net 10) (status 10))
 (segment (start 144.49651 76.073) (end 145.3255 75.24401) (width 0.25) (layer F.Cu) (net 8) (status 10))
 (segment (start 144.3 76.073) (end 144.49651 76.073) (width 0.25) (layer F.Cu) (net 8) (status 30))
 (segment (start 145.3255 75.24401) (end 146.1395 75.24401) (width 0.25) (layer F.Cu) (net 8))
 (segment (start 146.1395 75.24401) (end 146.48899 74.89452) (width 0.25) (layer F.Cu) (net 8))
 (segment (start 147.7515 72.233) (end 147.7515 72.883) (width 0.25) (layer F.Cu) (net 8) (status 30))
 (segment (start 146.48899 74.89452) (end 146.488991 74.405897) (width 0.25) (layer F.Cu) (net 8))
 (segment (start 146.488991 74.405897) (end 146.93899 73.955898) (width 0.25) (layer F.Cu) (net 8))
 (segment (start 147.264 72.883) (end 147.7515 72.883) (width 0.25) (layer F.Cu) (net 8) (status 30))
 (segment (start 146.93899 73.20801) (end 147.264 72.883) (width 0.25) (layer F.Cu) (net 8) (status 20))
 (segment (start 146.93899 73.955898) (end 146.93899 73.20801) (width 0.25) (layer F.Cu) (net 8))
 (segment (start 147.774 73.533) (end 147.774 74.183) (width 0.25) (layer F.Cu) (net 9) (status 30))
 (segment (start 147.348298 74.183) (end 146.939 74.592298) (width 0.25) (layer F.Cu) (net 9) (status 10))
 (segment (start 147.7515 74.183) (end 147.348298 74.183) (width 0.25) (layer F.Cu) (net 9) (status 30))
 (segment (start 146.448 76.073) (end 145.923 76.073) (width 0.25) (layer F.Cu) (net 9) (status 20))
 (segment (start 146.939 75.582) (end 146.448 76.073) (width 0.25) (layer F.Cu) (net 9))
 (segment (start 146.939 74.592298) (end 146.939 75.582) (width 0.25) (layer F.Cu) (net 9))
 (segment (start 143.786 77.746) (end 145.034 77.746) (width 0.5) (layer F.Cu) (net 4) (status 20))
 (segment (start 142.24 76.2) (end 143.786 77.746) (width 0.5) (layer F.Cu) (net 4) (status 10))
 (segment (start 147.7515 75.868788) (end 147.7515 74.833) (width 0.5) (layer F.Cu) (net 4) (status 20))
 (segment (start 145.874288 77.746) (end 147.7515 75.868788) (width 0.5) (layer F.Cu) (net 4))
 (segment (start 145.034 77.746) (end 145.874288 77.746) (width 0.5) (layer F.Cu) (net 4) (status 10))
 (segment (start 142.606 83.454) (end 142.24 83.82) (width 0.25) (layer F.Cu) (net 5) (status 30))
 (segment (start 143.525 85.105) (end 142.24 83.82) (width 0.3) (layer F.Cu) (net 5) (status 20))
 (segment (start 145.034 85.105) (end 143.525 85.105) (width 0.3) (layer F.Cu) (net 5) (status 10))
 (segment (start 145.034 85.105) (end 147.051 85.105) (width 0.3) (layer F.Cu) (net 5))
 (segment (start 150.764 81.392) (end 150.764 75.8955) (width 0.3) (layer F.Cu) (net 5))
 (segment (start 147.051 85.105) (end 150.764 81.392) (width 0.3) (layer F.Cu) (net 5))
 (segment (start 150.114 81.107692) (end 150.114 75.8955) (width 0.3) (layer F.Cu) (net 6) (status 20))
 (segment (start 147.416692 83.805) (end 150.114 81.107692) (width 0.3) (layer F.Cu) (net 6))
 (segment (start 145.034 83.805) (end 147.416692 83.805) (width 0.3) (layer F.Cu) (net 6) (status 10))
 (segment (start 145.034 82.282) (end 145.034 83.805) (width 0.3) (layer F.Cu) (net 6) (status 30))
 (segment (start 144.032 81.28) (end 145.034 82.282) (width 0.3) (layer F.Cu) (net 6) (status 20))
 (segment (start 142.24 81.28) (end 144.032 81.28) (width 0.3) (layer F.Cu) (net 6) (status 10))
 (segment (start 142.748 78.232) (end 142.24 78.74) (width 0.25) (layer F.Cu) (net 3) (status 30))
 (segment (start 147.066 82.707) (end 147.798 82.707) (width 0.3) (layer F.Cu) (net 3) (status 30))
 (segment (start 149.464 81.041) (end 149.464 75.804) (width 0.3) (layer F.Cu) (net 3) (status 20))
 (segment (start 147.798 82.707) (end 149.464 81.041) (width 0.3) (layer F.Cu) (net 3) (status 10))
 (segment (start 149.464 75.804) (end 149.464 75.8955) (width 0.3) (layer F.Cu) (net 3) (status 30))
 (segment (start 144.728 78.74) (end 145.034 79.046) (width 0.3) (layer F.Cu) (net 3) (status 30))
 (segment (start 142.24 78.74) (end 144.728 78.74) (width 0.3) (layer F.Cu) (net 3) (status 30))
 (segment (start 145.034 79.046) (end 145.034 80.532) (width 0.3) (layer F.Cu) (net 3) (status 30))
 (segment (start 145.965999 82.354591) (end 146.318408 82.707) (width 0.3) (layer F.Cu) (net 3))
 (segment (start 146.318408 82.707) (end 147.066 82.707) (width 0.3) (layer F.Cu) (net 3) (status 20))
 (segment (start 145.965999 80.988999) (end 145.965999 82.354591) (width 0.3) (layer F.Cu) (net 3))
 (segment (start 145.509 80.532) (end 145.965999 80.988999) (width 0.3) (layer F.Cu) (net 3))
 (segment (start 145.034 80.532) (end 145.509 80.532) (width 0.3) (layer F.Cu) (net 3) (status 10))
 (segment (start 148.814 75.8955) (end 148.814 76.043) (width 0.3) (layer F.Cu) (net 2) (status 30))
 (segment (start 148.814 76.043) (end 148.844 76.073) (width 0.3) (layer F.Cu) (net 2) (status 30))
 (segment (start 148.116 81.407) (end 147.066 81.407) (width 0.3) (layer F.Cu) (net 2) (status 20))
 (segment (start 148.844 76.073) (end 148.844 80.679) (width 0.3) (layer F.Cu) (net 2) (status 10))
 (segment (start 148.844 80.679) (end 148.116 81.407) (width 0.3) (layer F.Cu) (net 2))
 (segment (start 148.741 71.12) (end 148.814 71.193) (width 0.25) (layer F.Cu) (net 7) (status 30))
 (segment (start 145.669 71.374) (end 145.923 71.12) (width 0.25) (layer F.Cu) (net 7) (status 30))
 (segment (start 145.669 72.644) (end 145.669 71.374) (width 0.25) (layer F.Cu) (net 7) (status 30))
 (segment (start 147.124388 71.1705) (end 148.814 71.1705) (width 0.25) (layer F.Cu) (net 7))
 (segment (start 146.412888 71.882) (end 147.124388 71.1705) (width 0.25) (layer F.Cu) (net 7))
 (segment (start 145.669 72.644) (end 145.669 72.119) (width 0.25) (layer F.Cu) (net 7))
 (segment (start 145.906 71.882) (end 146.412888 71.882) (width 0.25) (layer F.Cu) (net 7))
 (segment (start 145.669 72.119) (end 145.906 71.882) (width 0.25) (layer F.Cu) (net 7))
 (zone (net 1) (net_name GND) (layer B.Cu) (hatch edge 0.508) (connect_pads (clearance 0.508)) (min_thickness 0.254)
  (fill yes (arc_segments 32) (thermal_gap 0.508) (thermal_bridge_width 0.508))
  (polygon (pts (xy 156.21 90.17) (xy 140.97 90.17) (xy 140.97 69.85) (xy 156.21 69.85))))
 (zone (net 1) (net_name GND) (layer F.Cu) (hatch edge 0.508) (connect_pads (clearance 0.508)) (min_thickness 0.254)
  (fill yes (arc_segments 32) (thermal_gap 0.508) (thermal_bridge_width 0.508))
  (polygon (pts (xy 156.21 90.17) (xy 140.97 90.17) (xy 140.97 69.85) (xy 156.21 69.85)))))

